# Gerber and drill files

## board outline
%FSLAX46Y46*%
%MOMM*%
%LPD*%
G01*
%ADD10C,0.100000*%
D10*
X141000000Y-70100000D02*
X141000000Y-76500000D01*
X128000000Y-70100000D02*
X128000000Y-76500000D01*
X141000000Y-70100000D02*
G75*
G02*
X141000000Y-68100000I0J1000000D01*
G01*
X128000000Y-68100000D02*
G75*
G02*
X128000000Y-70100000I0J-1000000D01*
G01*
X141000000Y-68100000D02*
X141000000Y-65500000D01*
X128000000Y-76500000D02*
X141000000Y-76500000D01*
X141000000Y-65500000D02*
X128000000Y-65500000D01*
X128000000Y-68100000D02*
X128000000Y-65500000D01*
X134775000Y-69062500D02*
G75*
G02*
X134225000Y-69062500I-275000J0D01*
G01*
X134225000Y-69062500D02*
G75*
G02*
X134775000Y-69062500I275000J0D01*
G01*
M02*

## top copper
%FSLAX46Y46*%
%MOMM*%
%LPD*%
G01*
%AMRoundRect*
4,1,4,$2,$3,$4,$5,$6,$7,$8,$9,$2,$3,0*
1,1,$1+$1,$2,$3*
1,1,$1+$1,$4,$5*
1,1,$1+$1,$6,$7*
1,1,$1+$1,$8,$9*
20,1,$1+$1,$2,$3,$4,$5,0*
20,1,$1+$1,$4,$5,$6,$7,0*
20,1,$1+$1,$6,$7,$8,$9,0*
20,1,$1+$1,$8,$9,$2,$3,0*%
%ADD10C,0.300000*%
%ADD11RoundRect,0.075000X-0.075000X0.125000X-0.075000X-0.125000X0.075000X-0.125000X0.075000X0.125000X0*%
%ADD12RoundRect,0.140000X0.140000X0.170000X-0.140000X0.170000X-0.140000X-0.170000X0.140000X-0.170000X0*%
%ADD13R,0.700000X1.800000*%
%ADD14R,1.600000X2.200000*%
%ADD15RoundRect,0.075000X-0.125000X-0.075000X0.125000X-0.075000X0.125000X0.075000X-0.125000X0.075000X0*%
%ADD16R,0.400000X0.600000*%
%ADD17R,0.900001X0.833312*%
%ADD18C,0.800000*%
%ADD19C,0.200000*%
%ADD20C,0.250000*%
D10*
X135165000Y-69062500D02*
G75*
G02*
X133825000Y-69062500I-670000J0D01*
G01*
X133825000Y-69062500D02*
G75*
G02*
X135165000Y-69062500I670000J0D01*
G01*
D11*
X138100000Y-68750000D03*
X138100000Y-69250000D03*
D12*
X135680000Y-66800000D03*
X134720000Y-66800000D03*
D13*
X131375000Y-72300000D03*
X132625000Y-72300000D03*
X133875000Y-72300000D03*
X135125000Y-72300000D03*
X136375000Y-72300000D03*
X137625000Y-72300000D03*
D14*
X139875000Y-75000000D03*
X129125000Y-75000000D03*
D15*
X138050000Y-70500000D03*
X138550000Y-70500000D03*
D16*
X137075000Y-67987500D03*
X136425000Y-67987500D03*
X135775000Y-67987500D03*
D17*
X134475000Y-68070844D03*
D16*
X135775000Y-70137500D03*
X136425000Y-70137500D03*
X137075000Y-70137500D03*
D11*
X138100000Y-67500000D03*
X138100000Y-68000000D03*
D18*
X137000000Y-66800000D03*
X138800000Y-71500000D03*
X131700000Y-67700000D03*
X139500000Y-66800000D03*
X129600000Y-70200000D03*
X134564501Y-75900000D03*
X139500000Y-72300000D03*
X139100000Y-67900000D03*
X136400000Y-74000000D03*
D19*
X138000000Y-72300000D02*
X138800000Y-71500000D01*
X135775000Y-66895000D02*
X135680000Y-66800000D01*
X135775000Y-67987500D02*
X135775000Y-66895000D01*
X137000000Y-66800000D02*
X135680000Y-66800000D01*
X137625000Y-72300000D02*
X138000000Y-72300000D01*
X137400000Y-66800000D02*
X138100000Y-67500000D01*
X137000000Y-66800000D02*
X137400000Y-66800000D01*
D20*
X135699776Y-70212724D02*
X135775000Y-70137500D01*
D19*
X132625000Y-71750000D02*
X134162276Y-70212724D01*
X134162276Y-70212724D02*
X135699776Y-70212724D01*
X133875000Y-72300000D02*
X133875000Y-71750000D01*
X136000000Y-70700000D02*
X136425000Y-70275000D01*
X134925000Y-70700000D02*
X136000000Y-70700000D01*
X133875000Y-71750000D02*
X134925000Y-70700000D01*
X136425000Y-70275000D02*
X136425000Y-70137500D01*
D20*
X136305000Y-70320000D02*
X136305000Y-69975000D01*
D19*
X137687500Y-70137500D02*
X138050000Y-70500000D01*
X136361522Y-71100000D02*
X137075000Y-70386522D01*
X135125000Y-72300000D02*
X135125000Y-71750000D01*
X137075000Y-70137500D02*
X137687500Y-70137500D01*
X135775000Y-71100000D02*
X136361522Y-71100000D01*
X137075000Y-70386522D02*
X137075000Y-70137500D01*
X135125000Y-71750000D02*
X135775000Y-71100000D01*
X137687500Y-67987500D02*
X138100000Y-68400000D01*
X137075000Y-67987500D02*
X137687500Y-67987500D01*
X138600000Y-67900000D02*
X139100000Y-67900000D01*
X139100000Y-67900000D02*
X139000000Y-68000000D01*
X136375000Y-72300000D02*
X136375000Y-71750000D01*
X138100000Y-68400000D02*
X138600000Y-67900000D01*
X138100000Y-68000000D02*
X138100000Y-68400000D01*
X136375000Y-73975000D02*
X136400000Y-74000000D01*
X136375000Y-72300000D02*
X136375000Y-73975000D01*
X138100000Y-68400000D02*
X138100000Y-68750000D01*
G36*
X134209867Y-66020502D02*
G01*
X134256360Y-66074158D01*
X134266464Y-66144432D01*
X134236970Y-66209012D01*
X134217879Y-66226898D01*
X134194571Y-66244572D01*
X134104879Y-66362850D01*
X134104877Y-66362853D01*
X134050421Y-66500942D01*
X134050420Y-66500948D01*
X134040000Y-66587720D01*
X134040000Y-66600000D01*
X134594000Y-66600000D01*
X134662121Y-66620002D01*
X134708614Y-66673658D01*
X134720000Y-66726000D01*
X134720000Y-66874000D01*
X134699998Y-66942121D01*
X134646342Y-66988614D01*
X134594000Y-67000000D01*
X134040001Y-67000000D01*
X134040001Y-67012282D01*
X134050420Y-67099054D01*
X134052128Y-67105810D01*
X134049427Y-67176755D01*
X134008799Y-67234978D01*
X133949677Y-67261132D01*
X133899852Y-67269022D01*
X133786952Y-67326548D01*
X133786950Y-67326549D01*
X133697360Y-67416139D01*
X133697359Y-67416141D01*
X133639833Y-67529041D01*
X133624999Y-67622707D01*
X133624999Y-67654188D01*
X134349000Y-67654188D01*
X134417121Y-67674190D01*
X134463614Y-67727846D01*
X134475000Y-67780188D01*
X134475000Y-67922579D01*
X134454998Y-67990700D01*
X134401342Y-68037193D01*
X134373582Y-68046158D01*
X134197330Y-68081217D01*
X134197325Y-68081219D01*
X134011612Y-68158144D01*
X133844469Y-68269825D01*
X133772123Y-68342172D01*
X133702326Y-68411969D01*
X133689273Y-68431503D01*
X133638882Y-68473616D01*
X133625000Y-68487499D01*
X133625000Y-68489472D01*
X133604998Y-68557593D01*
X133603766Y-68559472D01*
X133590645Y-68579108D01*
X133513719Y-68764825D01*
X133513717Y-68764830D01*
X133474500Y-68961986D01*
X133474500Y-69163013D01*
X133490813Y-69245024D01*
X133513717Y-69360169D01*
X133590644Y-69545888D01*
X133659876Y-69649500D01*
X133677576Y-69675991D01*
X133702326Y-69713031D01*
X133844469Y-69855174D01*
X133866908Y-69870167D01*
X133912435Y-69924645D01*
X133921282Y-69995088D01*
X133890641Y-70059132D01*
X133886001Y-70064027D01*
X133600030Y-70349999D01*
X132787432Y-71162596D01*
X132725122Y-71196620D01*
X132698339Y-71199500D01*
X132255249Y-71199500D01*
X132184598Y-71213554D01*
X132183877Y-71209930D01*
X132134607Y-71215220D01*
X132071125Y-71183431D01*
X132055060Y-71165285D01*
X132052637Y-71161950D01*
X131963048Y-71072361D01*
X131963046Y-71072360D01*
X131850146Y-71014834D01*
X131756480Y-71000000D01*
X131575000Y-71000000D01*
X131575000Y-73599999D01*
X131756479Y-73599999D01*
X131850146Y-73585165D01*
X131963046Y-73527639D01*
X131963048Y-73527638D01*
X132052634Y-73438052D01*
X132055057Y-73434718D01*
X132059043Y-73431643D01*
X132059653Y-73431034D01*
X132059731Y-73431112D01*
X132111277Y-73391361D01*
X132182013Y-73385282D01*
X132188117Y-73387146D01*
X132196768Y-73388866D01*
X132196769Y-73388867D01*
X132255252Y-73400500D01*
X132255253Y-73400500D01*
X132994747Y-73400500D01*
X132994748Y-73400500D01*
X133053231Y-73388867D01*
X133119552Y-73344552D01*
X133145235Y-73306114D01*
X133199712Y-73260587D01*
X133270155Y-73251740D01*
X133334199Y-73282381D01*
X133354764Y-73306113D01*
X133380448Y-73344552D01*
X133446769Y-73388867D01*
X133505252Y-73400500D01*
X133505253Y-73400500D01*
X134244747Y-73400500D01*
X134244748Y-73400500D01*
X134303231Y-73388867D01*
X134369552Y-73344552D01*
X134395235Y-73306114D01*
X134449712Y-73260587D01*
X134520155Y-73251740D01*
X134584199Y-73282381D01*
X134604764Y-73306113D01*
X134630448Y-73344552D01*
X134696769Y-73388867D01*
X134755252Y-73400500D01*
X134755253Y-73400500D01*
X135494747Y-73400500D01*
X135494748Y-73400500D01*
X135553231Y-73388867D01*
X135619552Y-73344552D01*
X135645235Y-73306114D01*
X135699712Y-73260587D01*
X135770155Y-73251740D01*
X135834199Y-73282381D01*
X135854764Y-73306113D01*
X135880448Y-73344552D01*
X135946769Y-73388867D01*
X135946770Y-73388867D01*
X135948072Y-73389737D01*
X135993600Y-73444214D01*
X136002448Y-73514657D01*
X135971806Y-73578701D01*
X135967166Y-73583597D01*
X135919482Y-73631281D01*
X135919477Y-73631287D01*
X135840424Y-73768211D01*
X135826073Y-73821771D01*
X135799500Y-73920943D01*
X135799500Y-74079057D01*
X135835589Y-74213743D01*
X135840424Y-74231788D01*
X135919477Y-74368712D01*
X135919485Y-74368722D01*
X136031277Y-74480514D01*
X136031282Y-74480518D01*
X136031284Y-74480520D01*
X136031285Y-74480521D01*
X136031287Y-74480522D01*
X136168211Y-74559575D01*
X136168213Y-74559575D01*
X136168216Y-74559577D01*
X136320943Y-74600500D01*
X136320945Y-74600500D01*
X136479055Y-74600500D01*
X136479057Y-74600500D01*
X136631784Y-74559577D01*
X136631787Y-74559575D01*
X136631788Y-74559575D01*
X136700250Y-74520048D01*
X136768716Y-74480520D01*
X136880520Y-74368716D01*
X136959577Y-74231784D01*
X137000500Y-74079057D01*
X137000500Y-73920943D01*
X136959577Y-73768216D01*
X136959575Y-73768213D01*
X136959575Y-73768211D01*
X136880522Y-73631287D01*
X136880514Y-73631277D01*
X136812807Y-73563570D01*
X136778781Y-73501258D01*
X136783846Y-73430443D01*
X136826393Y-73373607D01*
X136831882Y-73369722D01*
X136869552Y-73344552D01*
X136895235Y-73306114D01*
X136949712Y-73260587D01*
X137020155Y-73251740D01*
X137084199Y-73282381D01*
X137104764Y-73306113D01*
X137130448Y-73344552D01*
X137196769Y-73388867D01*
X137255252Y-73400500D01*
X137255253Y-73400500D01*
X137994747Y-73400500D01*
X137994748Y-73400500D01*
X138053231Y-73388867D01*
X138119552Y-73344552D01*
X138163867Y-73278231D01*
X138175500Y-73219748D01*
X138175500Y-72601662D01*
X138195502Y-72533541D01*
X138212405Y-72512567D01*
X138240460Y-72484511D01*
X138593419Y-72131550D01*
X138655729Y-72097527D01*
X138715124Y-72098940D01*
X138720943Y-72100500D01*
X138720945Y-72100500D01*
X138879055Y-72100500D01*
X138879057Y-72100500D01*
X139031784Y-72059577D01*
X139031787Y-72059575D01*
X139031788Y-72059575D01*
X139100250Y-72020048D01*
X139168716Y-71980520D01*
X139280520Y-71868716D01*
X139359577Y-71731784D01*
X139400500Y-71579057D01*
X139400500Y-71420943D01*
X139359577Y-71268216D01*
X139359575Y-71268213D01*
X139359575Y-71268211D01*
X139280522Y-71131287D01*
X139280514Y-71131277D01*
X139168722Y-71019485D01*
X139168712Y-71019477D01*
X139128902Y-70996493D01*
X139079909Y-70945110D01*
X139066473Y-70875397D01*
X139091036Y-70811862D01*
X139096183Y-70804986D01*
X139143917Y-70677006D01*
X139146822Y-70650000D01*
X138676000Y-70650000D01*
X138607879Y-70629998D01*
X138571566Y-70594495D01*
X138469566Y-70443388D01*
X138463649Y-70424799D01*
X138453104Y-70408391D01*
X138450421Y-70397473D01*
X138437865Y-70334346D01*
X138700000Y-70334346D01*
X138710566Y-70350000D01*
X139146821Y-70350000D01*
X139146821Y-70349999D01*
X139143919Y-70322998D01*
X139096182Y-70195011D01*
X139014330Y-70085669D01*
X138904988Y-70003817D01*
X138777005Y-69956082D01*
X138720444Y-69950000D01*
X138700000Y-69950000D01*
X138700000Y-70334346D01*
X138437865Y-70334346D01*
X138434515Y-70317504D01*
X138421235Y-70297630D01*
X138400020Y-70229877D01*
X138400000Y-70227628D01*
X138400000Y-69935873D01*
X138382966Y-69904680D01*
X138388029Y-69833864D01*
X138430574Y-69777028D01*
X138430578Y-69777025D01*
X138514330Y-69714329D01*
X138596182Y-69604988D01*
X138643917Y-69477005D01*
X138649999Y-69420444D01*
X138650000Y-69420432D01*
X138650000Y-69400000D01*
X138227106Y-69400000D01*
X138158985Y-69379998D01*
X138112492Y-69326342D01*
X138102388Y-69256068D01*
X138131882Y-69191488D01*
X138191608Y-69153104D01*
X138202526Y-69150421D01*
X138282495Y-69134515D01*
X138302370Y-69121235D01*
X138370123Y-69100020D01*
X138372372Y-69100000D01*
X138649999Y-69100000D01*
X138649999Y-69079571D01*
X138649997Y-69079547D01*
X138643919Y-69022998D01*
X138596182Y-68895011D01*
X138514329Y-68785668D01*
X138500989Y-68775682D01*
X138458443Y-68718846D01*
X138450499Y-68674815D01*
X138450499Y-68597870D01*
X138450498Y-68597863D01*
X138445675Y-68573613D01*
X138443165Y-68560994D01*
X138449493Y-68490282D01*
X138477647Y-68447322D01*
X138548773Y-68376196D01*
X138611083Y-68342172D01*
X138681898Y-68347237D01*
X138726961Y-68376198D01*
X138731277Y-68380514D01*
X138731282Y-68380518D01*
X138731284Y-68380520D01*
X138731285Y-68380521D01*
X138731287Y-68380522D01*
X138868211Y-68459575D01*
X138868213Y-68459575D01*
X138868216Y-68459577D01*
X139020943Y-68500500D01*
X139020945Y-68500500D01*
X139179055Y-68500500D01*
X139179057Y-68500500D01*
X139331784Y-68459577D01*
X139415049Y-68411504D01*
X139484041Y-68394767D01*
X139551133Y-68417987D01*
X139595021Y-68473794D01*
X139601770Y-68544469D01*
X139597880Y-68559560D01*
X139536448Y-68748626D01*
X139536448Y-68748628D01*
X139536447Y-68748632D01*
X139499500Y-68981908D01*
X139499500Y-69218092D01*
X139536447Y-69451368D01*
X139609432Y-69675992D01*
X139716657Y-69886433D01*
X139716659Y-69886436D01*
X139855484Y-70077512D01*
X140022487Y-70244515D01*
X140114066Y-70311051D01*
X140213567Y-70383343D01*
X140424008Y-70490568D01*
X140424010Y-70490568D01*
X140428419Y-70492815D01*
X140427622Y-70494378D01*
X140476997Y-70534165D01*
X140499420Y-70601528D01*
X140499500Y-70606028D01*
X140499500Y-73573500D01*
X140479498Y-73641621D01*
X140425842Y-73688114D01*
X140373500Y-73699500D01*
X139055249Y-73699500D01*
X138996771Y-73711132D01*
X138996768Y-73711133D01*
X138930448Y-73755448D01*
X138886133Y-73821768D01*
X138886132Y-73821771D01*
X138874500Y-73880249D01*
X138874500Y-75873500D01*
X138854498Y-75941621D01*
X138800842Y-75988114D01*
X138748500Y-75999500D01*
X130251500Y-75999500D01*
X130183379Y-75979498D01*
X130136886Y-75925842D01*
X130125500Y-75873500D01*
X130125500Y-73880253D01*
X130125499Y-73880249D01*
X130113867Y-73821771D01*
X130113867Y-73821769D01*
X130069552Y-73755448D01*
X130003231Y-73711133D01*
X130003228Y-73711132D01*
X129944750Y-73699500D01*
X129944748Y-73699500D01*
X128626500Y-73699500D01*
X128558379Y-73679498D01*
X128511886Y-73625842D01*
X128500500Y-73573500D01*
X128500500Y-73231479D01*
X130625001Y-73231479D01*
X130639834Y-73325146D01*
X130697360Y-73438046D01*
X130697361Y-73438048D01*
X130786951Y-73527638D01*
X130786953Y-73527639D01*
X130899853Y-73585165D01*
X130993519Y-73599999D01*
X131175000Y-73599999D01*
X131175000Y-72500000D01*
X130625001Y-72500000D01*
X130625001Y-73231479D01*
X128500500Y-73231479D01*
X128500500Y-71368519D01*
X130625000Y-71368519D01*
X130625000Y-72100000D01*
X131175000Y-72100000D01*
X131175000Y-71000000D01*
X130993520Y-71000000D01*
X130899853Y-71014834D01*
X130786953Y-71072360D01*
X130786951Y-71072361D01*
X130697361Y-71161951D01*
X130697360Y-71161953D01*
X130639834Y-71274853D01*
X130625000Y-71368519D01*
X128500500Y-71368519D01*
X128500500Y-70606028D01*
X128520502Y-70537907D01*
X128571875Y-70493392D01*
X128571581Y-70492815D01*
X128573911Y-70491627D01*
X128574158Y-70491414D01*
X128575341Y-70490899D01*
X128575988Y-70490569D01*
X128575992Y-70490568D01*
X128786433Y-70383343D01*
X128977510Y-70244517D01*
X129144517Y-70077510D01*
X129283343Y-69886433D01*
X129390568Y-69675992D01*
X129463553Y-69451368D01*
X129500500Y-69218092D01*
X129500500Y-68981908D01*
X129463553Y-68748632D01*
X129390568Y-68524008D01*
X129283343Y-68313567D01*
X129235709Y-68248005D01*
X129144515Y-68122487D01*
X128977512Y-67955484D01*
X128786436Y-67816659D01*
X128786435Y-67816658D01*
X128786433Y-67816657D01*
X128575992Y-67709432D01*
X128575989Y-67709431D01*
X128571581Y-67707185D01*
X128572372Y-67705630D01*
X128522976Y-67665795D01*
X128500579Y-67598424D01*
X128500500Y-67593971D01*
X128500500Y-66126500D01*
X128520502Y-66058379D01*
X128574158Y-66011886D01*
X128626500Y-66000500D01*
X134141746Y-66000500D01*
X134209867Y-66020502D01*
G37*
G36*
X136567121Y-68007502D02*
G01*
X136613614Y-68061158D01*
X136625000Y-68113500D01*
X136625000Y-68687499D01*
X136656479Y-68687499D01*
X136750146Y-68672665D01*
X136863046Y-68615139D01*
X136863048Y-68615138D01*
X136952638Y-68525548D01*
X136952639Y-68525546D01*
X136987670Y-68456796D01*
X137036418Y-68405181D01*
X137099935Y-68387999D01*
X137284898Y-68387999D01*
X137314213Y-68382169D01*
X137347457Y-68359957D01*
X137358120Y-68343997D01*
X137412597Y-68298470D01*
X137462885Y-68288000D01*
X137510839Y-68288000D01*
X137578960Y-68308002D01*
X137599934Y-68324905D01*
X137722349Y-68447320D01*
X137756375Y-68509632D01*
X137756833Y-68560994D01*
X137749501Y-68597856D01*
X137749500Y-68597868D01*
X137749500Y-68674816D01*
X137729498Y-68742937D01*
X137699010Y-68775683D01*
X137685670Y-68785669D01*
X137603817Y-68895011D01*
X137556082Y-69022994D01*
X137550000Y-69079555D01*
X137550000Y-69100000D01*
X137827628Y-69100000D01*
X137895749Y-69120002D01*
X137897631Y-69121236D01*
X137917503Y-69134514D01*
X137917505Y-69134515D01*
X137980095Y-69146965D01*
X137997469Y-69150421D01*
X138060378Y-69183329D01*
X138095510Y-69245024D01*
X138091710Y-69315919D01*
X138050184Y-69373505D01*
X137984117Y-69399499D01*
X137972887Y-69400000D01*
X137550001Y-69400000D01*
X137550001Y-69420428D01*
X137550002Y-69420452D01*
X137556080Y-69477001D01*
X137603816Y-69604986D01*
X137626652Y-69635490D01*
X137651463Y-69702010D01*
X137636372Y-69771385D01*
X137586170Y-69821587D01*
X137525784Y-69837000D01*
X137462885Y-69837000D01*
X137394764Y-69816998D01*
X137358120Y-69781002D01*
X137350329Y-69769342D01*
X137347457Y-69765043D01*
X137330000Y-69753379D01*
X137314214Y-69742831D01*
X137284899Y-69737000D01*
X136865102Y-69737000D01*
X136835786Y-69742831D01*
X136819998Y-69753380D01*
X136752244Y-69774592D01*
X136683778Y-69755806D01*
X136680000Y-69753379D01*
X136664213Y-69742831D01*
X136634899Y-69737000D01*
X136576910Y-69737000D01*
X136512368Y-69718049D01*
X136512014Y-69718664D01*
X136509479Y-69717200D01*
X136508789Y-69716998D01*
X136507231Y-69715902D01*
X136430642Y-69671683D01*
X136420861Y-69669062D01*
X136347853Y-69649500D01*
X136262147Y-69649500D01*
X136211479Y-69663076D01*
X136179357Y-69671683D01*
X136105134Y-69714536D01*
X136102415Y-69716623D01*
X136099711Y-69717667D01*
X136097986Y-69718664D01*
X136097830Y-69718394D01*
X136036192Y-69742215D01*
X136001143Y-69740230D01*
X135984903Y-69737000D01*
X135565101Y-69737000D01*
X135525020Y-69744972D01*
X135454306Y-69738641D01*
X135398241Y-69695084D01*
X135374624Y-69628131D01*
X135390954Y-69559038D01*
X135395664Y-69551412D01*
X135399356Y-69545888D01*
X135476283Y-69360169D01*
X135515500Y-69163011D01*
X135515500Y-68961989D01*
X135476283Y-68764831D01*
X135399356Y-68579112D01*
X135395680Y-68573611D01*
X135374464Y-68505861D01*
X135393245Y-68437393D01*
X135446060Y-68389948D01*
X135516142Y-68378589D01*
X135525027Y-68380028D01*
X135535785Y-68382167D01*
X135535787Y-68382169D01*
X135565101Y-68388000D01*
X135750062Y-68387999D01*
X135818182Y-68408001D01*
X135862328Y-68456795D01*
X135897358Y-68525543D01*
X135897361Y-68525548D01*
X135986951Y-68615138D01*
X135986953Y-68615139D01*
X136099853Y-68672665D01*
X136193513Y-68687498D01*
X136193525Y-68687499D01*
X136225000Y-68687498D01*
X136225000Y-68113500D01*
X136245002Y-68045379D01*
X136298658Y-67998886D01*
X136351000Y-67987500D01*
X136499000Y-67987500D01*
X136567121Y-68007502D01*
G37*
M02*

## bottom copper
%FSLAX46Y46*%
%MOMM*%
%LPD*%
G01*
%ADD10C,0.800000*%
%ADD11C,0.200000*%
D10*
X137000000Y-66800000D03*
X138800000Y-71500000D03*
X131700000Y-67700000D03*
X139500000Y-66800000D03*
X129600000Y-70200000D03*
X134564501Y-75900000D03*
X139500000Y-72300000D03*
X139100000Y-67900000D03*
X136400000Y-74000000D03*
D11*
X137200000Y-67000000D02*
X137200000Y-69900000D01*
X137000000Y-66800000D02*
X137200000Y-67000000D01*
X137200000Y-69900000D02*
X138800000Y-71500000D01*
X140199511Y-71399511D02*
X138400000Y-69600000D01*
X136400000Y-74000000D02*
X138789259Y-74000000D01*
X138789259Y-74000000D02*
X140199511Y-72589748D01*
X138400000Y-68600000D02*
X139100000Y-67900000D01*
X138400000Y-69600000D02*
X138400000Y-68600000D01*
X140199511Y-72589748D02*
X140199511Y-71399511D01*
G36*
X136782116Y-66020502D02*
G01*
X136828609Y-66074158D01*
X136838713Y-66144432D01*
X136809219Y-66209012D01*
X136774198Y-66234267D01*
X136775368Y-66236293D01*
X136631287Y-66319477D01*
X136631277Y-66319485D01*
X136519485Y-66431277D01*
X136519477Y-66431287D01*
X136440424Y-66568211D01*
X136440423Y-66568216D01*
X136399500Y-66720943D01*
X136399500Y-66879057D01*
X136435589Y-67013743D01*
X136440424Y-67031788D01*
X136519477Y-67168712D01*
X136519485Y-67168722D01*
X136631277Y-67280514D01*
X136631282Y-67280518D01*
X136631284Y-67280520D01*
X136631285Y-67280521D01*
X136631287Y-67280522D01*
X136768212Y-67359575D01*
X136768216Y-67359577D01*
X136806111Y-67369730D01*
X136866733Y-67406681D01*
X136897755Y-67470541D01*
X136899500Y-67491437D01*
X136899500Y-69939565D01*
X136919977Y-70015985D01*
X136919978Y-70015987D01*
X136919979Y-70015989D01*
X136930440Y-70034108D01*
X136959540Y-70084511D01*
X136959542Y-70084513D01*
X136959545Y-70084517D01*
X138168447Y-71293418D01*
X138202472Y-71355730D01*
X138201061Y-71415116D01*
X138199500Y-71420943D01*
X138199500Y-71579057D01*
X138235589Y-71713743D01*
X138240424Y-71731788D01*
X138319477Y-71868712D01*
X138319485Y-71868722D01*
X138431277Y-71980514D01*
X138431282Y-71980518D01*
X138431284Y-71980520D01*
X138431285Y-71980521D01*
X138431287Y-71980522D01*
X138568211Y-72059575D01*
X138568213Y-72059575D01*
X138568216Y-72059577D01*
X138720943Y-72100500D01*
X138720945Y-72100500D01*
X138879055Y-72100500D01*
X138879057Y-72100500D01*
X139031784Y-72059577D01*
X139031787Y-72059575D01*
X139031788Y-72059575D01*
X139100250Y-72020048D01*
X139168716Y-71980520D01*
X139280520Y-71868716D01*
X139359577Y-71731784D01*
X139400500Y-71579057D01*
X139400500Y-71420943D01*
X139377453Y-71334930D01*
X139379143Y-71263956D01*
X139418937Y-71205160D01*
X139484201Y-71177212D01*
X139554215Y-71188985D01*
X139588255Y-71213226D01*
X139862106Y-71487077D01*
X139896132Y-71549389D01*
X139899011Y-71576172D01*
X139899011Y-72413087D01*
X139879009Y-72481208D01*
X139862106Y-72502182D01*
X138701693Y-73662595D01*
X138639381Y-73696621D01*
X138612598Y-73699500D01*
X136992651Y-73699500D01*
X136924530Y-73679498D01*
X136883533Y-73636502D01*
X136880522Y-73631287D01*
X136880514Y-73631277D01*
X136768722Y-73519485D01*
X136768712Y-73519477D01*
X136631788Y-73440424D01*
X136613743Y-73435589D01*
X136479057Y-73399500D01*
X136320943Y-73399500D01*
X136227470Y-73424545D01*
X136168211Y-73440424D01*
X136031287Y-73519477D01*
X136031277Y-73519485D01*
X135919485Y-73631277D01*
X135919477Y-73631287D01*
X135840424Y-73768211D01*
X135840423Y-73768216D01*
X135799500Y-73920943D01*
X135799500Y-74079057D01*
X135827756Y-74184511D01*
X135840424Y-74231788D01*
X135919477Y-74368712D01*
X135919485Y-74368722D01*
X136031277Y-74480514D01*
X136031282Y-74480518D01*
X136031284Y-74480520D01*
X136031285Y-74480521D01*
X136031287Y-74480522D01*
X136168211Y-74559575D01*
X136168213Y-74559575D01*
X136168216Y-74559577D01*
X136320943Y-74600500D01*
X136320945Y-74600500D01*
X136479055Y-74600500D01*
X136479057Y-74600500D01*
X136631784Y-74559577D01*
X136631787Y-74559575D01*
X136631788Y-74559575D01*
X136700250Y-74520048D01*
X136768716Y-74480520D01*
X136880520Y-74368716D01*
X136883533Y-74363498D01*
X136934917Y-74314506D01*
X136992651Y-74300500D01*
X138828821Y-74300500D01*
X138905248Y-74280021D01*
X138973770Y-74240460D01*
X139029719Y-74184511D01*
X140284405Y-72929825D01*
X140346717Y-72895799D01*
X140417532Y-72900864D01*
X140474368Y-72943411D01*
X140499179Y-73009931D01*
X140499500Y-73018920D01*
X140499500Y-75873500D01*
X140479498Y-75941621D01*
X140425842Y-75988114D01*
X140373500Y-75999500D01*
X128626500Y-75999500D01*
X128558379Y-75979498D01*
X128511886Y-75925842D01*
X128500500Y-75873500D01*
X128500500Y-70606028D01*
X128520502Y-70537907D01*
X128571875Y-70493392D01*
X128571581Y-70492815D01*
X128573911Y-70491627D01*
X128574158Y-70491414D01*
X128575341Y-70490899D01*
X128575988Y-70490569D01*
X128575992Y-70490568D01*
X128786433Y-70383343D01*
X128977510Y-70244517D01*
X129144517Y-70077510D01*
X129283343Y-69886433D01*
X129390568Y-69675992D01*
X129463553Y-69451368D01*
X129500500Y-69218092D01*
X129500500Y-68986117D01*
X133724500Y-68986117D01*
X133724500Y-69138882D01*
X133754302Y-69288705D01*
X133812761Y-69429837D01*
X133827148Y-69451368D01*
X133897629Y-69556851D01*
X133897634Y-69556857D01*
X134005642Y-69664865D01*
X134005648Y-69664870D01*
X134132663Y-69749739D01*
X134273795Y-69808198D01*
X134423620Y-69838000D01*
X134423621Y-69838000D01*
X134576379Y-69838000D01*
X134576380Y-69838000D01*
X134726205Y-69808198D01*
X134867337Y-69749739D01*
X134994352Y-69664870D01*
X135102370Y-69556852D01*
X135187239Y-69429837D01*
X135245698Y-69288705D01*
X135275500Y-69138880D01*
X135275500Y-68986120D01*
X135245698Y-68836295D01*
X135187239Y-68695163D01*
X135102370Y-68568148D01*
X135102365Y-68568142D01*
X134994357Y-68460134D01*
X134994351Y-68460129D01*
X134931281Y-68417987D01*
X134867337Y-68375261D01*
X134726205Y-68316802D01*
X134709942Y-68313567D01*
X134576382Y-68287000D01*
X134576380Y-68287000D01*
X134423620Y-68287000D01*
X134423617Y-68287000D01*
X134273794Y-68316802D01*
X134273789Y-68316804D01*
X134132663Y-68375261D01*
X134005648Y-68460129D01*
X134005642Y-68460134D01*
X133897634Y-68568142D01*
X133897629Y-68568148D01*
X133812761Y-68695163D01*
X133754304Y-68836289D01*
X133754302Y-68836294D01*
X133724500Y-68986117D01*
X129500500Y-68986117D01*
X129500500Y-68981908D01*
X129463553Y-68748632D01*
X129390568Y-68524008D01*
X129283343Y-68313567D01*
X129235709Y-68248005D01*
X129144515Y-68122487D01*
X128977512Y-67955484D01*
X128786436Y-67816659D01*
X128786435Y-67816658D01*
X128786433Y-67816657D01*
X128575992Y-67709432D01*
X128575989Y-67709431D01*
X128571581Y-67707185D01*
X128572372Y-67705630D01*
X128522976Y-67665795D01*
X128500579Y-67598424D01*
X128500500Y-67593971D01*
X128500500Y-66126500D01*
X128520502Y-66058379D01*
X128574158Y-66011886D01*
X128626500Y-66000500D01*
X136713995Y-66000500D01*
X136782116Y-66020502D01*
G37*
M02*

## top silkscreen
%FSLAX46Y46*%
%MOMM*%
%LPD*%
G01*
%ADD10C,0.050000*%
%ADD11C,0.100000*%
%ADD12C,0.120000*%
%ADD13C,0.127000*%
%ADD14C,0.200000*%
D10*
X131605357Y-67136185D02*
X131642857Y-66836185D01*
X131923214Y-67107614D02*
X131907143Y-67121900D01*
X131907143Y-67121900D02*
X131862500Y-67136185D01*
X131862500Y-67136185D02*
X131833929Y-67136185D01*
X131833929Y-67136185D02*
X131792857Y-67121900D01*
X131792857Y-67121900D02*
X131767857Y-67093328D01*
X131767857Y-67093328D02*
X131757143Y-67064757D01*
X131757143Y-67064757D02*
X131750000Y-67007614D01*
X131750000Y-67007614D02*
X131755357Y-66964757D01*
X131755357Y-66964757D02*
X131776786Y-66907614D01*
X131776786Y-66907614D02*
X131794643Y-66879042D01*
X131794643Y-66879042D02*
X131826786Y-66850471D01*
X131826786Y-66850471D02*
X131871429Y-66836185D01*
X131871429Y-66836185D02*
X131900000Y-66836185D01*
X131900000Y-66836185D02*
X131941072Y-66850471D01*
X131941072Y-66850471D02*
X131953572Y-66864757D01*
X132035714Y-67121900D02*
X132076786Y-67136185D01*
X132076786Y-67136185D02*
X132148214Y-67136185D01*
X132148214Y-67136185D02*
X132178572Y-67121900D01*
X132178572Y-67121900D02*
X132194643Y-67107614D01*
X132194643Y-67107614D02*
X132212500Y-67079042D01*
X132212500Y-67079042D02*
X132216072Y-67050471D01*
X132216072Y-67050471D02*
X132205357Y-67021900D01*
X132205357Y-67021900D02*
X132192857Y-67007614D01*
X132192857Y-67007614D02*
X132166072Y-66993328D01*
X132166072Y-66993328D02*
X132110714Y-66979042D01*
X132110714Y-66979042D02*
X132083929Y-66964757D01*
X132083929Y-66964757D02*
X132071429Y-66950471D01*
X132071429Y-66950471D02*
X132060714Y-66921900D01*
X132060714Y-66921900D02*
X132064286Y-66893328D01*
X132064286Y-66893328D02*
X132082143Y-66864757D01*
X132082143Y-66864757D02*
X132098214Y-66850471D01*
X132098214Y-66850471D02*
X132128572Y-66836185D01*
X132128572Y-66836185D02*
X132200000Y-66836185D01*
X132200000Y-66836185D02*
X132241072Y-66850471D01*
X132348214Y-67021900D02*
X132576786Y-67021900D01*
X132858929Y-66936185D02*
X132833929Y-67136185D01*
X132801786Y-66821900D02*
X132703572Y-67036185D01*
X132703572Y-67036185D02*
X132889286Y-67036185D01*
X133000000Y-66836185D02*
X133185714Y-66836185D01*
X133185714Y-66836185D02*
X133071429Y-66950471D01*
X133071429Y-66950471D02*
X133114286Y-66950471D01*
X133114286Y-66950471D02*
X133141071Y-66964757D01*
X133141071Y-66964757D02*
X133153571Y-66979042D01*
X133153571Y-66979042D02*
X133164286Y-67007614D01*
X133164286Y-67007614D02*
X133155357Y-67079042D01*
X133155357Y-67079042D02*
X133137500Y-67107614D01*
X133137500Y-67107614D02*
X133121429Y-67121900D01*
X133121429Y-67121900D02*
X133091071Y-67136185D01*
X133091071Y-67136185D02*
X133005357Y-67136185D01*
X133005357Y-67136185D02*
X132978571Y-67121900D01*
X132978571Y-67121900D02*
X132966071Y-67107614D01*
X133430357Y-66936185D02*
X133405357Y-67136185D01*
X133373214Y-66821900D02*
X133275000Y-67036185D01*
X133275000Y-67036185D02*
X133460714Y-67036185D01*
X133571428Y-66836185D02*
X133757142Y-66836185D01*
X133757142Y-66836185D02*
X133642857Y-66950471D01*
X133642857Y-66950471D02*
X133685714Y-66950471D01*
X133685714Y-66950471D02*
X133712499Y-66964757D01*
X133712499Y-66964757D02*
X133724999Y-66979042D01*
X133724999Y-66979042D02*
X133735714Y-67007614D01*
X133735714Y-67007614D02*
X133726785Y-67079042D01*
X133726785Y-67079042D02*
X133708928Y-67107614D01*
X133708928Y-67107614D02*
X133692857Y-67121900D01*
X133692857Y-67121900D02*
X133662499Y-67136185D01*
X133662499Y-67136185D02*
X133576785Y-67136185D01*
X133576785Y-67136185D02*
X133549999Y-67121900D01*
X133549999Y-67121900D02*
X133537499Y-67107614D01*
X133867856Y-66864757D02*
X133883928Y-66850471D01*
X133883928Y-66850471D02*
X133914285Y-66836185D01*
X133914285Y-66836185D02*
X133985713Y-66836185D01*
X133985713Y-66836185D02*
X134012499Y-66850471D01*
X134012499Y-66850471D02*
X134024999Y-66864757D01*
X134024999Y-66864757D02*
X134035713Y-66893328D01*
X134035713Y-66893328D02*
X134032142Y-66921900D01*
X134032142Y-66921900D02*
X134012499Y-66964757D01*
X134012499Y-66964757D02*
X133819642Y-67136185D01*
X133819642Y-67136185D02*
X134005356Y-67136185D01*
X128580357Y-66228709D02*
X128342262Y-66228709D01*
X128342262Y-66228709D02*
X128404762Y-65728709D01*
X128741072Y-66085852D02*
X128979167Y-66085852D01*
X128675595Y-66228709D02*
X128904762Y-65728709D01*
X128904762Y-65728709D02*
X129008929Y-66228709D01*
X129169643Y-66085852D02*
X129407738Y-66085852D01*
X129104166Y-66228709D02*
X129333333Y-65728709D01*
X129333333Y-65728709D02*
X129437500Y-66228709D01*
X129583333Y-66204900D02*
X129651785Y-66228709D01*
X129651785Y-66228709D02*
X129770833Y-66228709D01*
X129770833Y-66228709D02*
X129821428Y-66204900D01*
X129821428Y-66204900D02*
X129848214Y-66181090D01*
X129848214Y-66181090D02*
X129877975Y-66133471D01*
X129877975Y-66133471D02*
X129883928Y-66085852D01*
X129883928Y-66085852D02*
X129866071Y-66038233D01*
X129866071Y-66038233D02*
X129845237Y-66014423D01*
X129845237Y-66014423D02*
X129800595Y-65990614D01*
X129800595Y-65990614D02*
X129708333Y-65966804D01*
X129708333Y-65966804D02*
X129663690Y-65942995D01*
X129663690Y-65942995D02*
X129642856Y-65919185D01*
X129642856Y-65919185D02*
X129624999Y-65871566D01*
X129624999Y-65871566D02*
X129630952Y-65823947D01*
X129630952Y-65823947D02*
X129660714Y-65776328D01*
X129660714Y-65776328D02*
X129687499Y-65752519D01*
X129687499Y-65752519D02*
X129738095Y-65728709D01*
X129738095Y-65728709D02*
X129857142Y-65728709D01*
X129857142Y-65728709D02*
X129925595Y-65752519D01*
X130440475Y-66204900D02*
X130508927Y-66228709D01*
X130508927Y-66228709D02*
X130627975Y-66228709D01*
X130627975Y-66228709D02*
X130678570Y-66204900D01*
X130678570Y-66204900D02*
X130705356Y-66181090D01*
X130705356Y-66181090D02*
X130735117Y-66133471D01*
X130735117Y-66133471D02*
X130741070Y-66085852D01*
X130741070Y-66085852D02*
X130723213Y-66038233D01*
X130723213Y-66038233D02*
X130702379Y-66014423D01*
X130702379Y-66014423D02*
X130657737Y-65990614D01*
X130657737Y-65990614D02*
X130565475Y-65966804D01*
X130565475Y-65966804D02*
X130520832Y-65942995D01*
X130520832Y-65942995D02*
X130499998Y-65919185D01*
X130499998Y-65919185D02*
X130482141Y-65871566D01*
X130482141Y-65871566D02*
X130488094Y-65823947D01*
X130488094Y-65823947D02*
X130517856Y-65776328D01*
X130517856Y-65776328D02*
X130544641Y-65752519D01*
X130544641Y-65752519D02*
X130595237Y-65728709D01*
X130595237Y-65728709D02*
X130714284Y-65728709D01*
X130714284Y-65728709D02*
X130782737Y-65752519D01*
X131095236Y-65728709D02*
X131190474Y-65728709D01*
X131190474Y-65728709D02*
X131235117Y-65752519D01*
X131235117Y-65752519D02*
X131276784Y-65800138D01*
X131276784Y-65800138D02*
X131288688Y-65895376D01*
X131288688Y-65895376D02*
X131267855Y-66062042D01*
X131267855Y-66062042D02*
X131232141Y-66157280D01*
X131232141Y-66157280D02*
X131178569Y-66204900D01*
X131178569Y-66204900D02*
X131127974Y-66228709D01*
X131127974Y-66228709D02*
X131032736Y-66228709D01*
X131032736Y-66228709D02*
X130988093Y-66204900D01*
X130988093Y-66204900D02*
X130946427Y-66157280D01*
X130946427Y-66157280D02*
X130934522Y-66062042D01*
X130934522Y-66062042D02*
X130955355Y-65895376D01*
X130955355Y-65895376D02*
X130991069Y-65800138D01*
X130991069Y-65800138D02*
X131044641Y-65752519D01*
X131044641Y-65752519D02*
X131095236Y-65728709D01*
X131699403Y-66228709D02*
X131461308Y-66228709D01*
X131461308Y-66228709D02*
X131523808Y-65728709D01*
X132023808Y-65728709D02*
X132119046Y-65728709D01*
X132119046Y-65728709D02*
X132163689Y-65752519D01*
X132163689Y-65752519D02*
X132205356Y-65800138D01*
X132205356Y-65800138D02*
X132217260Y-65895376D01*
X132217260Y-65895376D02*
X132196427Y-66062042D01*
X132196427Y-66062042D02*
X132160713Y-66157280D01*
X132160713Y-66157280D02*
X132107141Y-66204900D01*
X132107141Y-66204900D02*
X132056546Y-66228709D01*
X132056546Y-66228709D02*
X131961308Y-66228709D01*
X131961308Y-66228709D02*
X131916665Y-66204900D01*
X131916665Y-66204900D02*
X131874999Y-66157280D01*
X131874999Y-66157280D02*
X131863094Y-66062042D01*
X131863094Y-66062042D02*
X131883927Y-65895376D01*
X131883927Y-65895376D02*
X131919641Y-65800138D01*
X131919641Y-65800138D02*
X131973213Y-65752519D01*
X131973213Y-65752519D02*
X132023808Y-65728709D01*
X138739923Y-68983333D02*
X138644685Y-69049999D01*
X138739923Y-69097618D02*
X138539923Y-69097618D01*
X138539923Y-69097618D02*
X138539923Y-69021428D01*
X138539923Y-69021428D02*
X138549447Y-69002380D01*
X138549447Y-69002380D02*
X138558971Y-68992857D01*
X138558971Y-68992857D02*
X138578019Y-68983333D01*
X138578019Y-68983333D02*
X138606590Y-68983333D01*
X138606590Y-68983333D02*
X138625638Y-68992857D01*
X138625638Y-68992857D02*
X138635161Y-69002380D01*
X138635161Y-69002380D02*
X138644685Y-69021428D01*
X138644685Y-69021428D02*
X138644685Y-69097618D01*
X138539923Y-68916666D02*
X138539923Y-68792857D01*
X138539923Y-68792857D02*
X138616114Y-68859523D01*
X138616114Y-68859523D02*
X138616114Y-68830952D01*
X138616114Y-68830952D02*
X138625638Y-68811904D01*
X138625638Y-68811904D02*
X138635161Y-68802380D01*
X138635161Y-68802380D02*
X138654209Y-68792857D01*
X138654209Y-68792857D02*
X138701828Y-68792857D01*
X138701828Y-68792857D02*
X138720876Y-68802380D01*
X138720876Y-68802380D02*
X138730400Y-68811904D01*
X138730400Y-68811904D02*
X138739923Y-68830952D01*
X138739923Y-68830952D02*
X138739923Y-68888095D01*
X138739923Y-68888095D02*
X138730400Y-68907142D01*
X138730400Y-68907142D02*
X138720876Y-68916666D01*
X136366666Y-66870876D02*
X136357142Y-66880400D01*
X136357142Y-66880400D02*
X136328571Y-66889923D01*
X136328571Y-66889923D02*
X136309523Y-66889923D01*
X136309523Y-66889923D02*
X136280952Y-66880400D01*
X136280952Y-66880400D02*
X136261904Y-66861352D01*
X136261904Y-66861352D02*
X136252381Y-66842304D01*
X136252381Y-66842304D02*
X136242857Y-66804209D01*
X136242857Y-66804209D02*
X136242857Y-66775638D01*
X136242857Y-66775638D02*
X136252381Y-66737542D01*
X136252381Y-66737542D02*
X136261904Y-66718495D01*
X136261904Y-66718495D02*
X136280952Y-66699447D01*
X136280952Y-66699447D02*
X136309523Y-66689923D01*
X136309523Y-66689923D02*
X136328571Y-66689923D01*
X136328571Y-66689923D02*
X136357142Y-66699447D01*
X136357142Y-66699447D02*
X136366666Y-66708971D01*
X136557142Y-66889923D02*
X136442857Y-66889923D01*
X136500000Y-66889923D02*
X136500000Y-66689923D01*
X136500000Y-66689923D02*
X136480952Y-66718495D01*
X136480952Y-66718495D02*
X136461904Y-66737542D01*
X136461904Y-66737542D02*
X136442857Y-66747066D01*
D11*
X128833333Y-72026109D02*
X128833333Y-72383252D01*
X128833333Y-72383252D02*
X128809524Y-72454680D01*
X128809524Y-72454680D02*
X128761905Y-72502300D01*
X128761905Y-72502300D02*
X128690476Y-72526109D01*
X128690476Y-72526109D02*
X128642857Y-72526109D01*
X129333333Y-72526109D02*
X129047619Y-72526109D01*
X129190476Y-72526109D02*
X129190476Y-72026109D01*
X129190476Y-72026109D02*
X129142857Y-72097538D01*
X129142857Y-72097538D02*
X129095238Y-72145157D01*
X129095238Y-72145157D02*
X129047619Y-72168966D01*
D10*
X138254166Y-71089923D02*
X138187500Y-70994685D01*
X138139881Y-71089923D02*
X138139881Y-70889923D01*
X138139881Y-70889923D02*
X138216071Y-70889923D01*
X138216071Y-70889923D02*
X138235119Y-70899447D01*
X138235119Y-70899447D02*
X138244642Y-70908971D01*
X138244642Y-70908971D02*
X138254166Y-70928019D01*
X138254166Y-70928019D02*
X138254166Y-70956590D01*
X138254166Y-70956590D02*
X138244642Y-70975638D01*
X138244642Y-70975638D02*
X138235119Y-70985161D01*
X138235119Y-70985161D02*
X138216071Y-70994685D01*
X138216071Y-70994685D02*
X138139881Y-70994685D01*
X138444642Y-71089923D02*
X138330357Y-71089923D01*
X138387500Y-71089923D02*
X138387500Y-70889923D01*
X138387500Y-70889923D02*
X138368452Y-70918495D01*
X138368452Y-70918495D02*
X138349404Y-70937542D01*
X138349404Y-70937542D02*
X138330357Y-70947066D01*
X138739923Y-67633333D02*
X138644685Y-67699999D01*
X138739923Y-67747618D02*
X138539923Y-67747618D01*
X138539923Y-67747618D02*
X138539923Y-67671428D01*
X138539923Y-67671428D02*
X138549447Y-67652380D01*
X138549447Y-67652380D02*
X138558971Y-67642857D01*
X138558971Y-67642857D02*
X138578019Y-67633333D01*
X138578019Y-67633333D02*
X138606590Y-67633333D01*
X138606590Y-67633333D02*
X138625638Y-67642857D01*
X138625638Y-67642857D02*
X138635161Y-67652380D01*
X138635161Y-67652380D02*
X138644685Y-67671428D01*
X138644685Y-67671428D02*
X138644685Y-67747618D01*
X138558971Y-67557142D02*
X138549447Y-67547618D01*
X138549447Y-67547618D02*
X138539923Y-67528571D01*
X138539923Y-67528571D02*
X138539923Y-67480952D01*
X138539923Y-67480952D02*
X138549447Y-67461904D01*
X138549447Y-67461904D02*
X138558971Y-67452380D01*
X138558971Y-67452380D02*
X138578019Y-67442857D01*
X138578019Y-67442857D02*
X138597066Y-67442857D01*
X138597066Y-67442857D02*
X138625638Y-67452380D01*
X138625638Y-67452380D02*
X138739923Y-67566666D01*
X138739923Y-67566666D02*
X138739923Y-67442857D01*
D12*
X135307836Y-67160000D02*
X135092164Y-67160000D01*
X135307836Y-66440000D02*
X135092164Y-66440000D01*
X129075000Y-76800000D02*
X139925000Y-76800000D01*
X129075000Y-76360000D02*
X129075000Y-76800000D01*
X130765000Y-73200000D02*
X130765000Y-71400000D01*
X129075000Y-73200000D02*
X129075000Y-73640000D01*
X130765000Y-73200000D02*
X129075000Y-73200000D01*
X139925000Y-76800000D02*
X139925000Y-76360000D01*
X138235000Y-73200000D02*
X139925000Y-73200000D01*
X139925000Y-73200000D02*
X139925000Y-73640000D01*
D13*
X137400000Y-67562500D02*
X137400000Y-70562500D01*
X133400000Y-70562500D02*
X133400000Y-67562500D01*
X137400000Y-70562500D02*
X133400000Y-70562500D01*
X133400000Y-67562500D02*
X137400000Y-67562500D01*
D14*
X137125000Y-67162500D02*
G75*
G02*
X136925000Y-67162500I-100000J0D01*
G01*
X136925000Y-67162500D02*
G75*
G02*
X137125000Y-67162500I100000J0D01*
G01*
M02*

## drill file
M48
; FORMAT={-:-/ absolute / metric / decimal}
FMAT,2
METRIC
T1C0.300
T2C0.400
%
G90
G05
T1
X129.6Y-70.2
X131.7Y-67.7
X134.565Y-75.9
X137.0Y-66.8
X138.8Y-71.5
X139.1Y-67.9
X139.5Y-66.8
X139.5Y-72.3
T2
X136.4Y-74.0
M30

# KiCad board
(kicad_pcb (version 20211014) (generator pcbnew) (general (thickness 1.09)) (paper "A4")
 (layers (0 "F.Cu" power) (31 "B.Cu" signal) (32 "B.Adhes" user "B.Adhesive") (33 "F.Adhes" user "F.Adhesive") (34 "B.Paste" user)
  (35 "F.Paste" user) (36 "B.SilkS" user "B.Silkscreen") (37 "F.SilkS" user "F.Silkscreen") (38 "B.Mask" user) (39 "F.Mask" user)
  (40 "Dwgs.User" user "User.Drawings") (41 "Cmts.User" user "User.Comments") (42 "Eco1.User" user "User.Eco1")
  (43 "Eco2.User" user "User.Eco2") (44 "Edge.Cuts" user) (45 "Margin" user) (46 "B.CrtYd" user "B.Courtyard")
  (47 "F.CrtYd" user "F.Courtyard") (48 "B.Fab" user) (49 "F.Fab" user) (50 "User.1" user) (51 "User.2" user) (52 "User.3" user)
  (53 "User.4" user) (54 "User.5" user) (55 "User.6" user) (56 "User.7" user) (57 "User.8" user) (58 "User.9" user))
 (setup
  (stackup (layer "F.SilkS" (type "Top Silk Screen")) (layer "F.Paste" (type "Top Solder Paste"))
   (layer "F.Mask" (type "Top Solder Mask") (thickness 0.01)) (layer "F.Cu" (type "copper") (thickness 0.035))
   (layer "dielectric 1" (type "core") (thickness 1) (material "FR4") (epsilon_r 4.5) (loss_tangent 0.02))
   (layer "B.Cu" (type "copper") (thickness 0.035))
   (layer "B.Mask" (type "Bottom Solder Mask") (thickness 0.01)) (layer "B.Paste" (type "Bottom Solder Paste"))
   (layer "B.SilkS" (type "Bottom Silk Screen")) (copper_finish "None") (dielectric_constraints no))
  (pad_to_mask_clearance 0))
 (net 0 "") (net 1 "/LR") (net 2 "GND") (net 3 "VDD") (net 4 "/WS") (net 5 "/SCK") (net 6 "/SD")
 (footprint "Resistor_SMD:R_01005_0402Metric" (layer "F.Cu") (at 138.1 69 -90)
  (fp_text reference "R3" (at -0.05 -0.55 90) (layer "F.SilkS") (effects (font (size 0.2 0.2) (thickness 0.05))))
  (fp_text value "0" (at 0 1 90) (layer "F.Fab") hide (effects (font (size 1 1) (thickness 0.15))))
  (pad "" smd roundrect (at -0.275 0 270) (size 0.27 0.27) (layers "F.Paste") (roundrect_rratio 0.25))
  (pad "" smd roundrect (at 0.275 0 270) (size 0.27 0.27) (layers "F.Paste") (roundrect_rratio 0.25))
  (pad "1" smd roundrect (at -0.25 0 270) (size 0.4 0.3) (layers "F.Cu" "F.Mask") (roundrect_rratio 0.25) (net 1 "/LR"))
  (pad "2" smd roundrect (at 0.25 0 270) (size 0.4 0.3) (layers "F.Cu" "F.Mask") (roundrect_rratio 0.25) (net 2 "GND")))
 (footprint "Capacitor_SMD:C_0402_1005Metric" (layer "F.Cu") (at 135.2 66.8 180)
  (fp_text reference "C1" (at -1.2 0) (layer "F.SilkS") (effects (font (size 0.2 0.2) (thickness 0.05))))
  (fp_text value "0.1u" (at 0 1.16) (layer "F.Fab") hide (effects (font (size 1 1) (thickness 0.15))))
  (fp_line (start -0.107836 -0.36) (end 0.107836 -0.36) (layer "F.SilkS") (width 0.12))
  (fp_line (start -0.107836 0.36) (end 0.107836 0.36) (layer "F.SilkS") (width 0.12))
  (pad "1" smd roundrect (at -0.48 0 180) (size 0.56 0.62) (layers "F.Cu" "F.Paste" "F.Mask") (roundrect_rratio 0.25) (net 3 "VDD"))
  (pad "2" smd roundrect (at 0.48 0 180) (size 0.56 0.62) (layers "F.Cu" "F.Paste" "F.Mask") (roundrect_rratio 0.25) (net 2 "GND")))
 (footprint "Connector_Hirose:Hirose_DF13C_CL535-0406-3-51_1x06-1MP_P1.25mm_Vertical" (layer "F.Cu") (at 134.5 73.75)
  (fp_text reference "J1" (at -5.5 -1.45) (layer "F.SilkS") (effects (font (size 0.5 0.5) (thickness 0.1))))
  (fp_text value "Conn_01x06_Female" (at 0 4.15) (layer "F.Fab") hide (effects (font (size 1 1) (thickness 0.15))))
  (fp_line (start -5.425 3.05) (end 5.425 3.05) (layer "F.SilkS") (width 0.12))
  (fp_line (start -5.425 2.61) (end -5.425 3.05) (layer "F.SilkS") (width 0.12))
  (fp_line (start -3.735 -0.55) (end -3.735 -2.35) (layer "F.SilkS") (width 0.12))
  (fp_line (start -5.425 -0.55) (end -5.425 -0.11) (layer "F.SilkS") (width 0.12))
  (fp_line (start -3.735 -0.55) (end -5.425 -0.55) (layer "F.SilkS") (width 0.12))
  (fp_line (start 5.425 3.05) (end 5.425 2.61) (layer "F.SilkS") (width 0.12))
  (fp_line (start 3.735 -0.55) (end 5.425 -0.55) (layer "F.SilkS") (width 0.12))
  (fp_line (start 5.425 -0.55) (end 5.425 -0.11) (layer "F.SilkS") (width 0.12))
  (pad "1" smd rect locked (at -3.125 -1.45) (size 0.7 1.8) (layers "F.Cu" "F.Paste" "F.Mask") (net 2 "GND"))
  (pad "2" smd rect locked (at -1.875 -1.45) (size 0.7 1.8) (layers "F.Cu" "F.Paste" "F.Mask") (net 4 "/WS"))
  (pad "3" smd rect locked (at -0.625 -1.45) (size 0.7 1.8) (layers "F.Cu" "F.Paste" "F.Mask") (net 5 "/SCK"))
  (pad "4" smd rect locked (at 0.625 -1.45) (size 0.7 1.8) (layers "F.Cu" "F.Paste" "F.Mask") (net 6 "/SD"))
  (pad "5" smd rect locked (at 1.875 -1.45) (size 0.7 1.8) (layers "F.Cu" "F.Paste" "F.Mask") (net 1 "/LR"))
  (pad "6" smd rect locked (at 3.125 -1.45) (size 0.7 1.8) (layers "F.Cu" "F.Paste" "F.Mask") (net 3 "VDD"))
  (pad "MP" smd rect locked (at 5.375 1.25) (size 1.6 2.2) (layers "F.Cu" "F.Paste" "F.Mask"))
  (pad "MP" smd rect locked (at -5.375 1.25) (size 1.6 2.2) (layers "F.Cu" "F.Paste" "F.Mask")))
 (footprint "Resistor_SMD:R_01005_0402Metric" (layer "F.Cu") (at 138.3 70.5)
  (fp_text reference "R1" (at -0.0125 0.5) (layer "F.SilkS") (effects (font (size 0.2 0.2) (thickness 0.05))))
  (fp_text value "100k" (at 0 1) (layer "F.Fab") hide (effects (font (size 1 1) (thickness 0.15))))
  (pad "" smd roundrect (at -0.275 0) (size 0.27 0.27) (layers "F.Paste") (roundrect_rratio 0.25))
  (pad "" smd roundrect (at 0.275 0) (size 0.27 0.27) (layers "F.Paste") (roundrect_rratio 0.25))
  (pad "1" smd roundrect (at -0.25 0) (size 0.4 0.3) (layers "F.Cu" "F.Mask") (roundrect_rratio 0.25) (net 6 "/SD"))
  (pad "2" smd roundrect (at 0.25 0) (size 0.4 0.3) (layers "F.Cu" "F.Mask") (roundrect_rratio 0.25) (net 2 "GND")))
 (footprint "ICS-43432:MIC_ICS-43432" (layer "F.Cu") (at 135.4 69.0625 -90) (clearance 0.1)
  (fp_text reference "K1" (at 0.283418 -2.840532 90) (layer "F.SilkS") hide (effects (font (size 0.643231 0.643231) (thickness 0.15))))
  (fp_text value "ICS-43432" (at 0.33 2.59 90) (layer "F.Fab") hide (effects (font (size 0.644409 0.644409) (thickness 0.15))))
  (fp_circle (center 0 0.905) (end 0.67 0.905) (layer "F.Cu") (width 0.3) (fill none))
  (fp_line (start -1.5 -2) (end 1.5 -2) (layer "F.SilkS") (width 0.127))
  (fp_line (start 1.5 2) (end -1.5 2) (layer "F.SilkS") (width 0.127))
  (fp_line (start 1.5 -2) (end 1.5 2) (layer "F.SilkS") (width 0.127))
  (fp_line (start -1.5 2) (end -1.5 -2) (layer "F.SilkS") (width 0.127))
  (fp_circle (center -1.9 -1.625) (end -1.8 -1.625) (layer "F.SilkS") (width 0.2) (fill none))
  (fp_circle (center 0 0.9) (end 0.275 0.9) (layer "Edge.Cuts") (width 0.1) (fill none))
  (pad "1" smd rect (at -1.075 -1.675 270) (size 0.6 0.4) (layers "F.Cu" "F.Mask") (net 1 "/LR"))
  (pad "2" smd rect (at -1.075 -1.025 270) (size 0.6 0.4) (layers "F.Cu" "F.Mask") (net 2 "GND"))
  (pad "3" smd rect (at -1.075 -0.375 270) (size 0.6 0.4) (layers "F.Cu" "F.Mask") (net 3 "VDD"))
  (pad "4" smd rect (at -0.991656 0.925 270) (size 0.833312 0.900001) (layers "F.Cu") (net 2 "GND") (thermal_width 1))
  (pad "5" smd rect (at 1.075 -0.375 270) (size 0.6 0.4) (layers "F.Cu" "F.Mask") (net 4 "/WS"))
  (pad "6" smd rect (at 1.075 -1.025 270) (size 0.6 0.4) (layers "F.Cu" "F.Mask") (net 5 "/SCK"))
  (pad "7" smd rect (at 1.075 -1.675 270) (size 0.6 0.4) (layers "F.Cu" "F.Mask") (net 6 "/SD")))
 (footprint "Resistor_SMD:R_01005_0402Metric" (layer "F.Cu") (at 138.1 67.75 -90)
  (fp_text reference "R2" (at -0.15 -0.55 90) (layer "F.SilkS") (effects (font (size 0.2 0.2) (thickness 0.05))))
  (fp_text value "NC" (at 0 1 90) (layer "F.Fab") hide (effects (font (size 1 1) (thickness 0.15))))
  (pad "" smd roundrect (at -0.275 0 270) (size 0.27 0.27) (layers "F.Paste") (roundrect_rratio 0.25))
  (pad "" smd roundrect (at 0.275 0 270) (size 0.27 0.27) (layers "F.Paste") (roundrect_rratio 0.25))
  (pad "1" smd roundrect (at -0.25 0 270) (size 0.4 0.3) (layers "F.Cu" "F.Mask") (roundrect_rratio 0.25) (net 3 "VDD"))
  (pad "2" smd roundrect (at 0.25 0 270) (size 0.4 0.3) (layers "F.Cu" "F.Mask") (roundrect_rratio 0.25) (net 1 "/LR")))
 (gr_line (start 141 70.1) (end 141 76.5) (layer "Edge.Cuts") (width 0.1))
 (gr_line (start 128 70.1) (end 128 76.5) (layer "Edge.Cuts") (width 0.1))
 (gr_arc (start 141 70.1) (mid 140 69.1) (end 141 68.1) (layer "Edge.Cuts") (width 0.1))
 (gr_arc (start 128 68.1) (mid 129 69.1) (end 128 70.1) (layer "Edge.Cuts") (width 0.1))
 (gr_line (start 141 68.1) (end 141 65.5) (layer "Edge.Cuts") (width 0.1))
 (gr_line (start 128 76.5) (end 141 76.5) (layer "Edge.Cuts") (width 0.1))
 (gr_line (start 141 65.5) (end 128 65.5) (layer "Edge.Cuts") (width 0.1))
 (gr_line (start 128 68.1) (end 128 65.5) (layer "Edge.Cuts") (width 0.1))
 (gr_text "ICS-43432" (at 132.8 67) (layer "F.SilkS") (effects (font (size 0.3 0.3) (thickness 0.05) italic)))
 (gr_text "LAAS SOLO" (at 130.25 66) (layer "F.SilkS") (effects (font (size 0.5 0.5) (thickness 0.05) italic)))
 (segment (start 138 72.3) (end 138.8 71.5) (width 0.2) (layer "F.Cu") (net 3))
 (segment (start 135.775 66.895) (end 135.68 66.8) (width 0.2) (layer "F.Cu") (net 3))
 (segment (start 135.775 67.9875) (end 135.775 66.895) (width 0.2) (layer "F.Cu") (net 3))
 (segment (start 137 66.8) (end 135.68 66.8) (width 0.2) (layer "F.Cu") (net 3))
 (segment (start 137.625 72.3) (end 138 72.3) (width 0.2) (layer "F.Cu") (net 3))
 (segment (start 137.4 66.8) (end 138.1 67.5) (width 0.2) (layer "F.Cu") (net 3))
 (segment (start 137 66.8) (end 137.4 66.8) (width 0.2) (layer "F.Cu") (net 3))
 (via (at 137 66.8) (size 0.8) (drill 0.3) (layers "F.Cu" "B.Cu") (free) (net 3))
 (via (at 138.8 71.5) (size 0.8) (drill 0.3) (layers "F.Cu" "B.Cu") (free) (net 3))
 (segment (start 137.2 67) (end 137.2 69.9) (width 0.2) (layer "B.Cu") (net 3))
 (segment (start 137 66.8) (end 137.2 67) (width 0.2) (layer "B.Cu") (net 3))
 (segment (start 137.2 69.9) (end 138.8 71.5) (width 0.2) (layer "B.Cu") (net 3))
 (via (at 131.7 67.7) (size 0.8) (drill 0.3) (layers "F.Cu" "B.Cu") (free) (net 2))
 (via (at 139.5 66.8) (size 0.8) (drill 0.3) (layers "F.Cu" "B.Cu") (free) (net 2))
 (via (at 129.6 70.2) (size 0.8) (drill 0.3) (layers "F.Cu" "B.Cu") (free) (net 2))
 (via (at 134.564501 75.9) (size 0.8) (drill 0.3) (layers "F.Cu" "B.Cu") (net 2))
 (via (at 139.5 72.3) (size 0.8) (drill 0.3) (layers "F.Cu" "B.Cu") (free) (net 2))
 (segment (start 135.699776 70.212724) (end 135.775 70.1375) (width 0.25) (layer "F.Cu") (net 4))
 (segment (start 132.625 71.75) (end 134.162276 70.212724) (width 0.2) (layer "F.Cu") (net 4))
 (segment (start 134.162276 70.212724) (end 135.699776 70.212724) (width 0.2) (layer "F.Cu") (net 4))
 (segment (start 133.875 72.3) (end 133.875 71.75) (width 0.2) (layer "F.Cu") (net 5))
 (segment (start 136 70.7) (end 136.425 70.275) (width 0.2) (layer "F.Cu") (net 5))
 (segment (start 134.925 70.7) (end 136 70.7) (width 0.2) (layer "F.Cu") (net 5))
 (segment (start 133.875 71.75) (end 134.925 70.7) (width 0.2) (layer "F.Cu") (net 5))
 (segment (start 136.425 70.275) (end 136.425 70.1375) (width 0.2) (layer "F.Cu") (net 5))
 (segment (start 136.305 70.32) (end 136.305 69.975) (width 0.25) (layer "F.Cu") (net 5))
 (segment (start 137.6875 70.1375) (end 138.05 70.5) (width 0.2) (layer "F.Cu") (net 6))
 (segment (start 136.361522 71.1) (end 137.075 70.386522) (width 0.2) (layer "F.Cu") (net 6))
 (segment (start 135.125 72.3) (end 135.125 71.75) (width 0.2) (layer "F.Cu") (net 6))
 (segment (start 137.075 70.1375) (end 137.6875 70.1375) (width 0.2) (layer "F.Cu") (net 6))
 (segment (start 135.775 71.1) (end 136.361522 71.1) (width 0.2) (layer "F.Cu") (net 6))
 (segment (start 137.075 70.386522) (end 137.075 70.1375) (width 0.2) (layer "F.Cu") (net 6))
 (segment (start 135.125 71.75) (end 135.775 71.1) (width 0.2) (layer "F.Cu") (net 6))
 (segment (start 137.6875 67.9875) (end 138.1 68.4) (width 0.2) (layer "F.Cu") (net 1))
 (segment (start 137.075 67.9875) (end 137.6875 67.9875) (width 0.2) (layer "F.Cu") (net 1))
 (segment (start 138.6 67.9) (end 139.1 67.9) (width 0.2) (layer "F.Cu") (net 1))
 (segment (start 139.1 67.9) (end 139 68) (width 0.2) (layer "F.Cu") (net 1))
 (segment (start 136.375 72.3) (end 136.375 71.75) (width 0.2) (layer "F.Cu") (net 1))
 (segment (start 138.1 68.4) (end 138.6 67.9) (width 0.2) (layer "F.Cu") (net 1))
 (segment (start 138.1 68) (end 138.1 68.4) (width 0.2) (layer "F.Cu") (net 1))
 (segment (start 136.375 73.975) (end 136.4 74) (width 0.2) (layer "F.Cu") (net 1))
 (segment (start 136.375 72.3) (end 136.375 73.975) (width 0.2) (layer "F.Cu") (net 1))
 (segment (start 138.1 68.4) (end 138.1 68.75) (width 0.2) (layer "F.Cu") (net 1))
 (via (at 139.1 67.9) (size 0.8) (drill 0.3) (layers "F.Cu" "B.Cu") (free) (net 1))
 (via (at 136.4 74) (size 0.8) (drill 0.4) (layers "F.Cu" "B.Cu") (free) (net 1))
 (segment (start 140.199511 71.399511) (end 138.4 69.6) (width 0.2) (layer "B.Cu") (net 1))
 (segment (start 136.4 74) (end 138.789259 74) (width 0.2) (layer "B.Cu") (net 1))
 (segment (start 138.789259 74) (end 140.199511 72.589748) (width 0.2) (layer "B.Cu") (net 1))
 (segment (start 138.4 68.6) (end 139.1 67.9) (width 0.2) (layer "B.Cu") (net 1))
 (segment (start 138.4 69.6) (end 138.4 68.6) (width 0.2) (layer "B.Cu") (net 1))
 (segment (start 140.199511 72.589748) (end 140.199511 71.399511) (width 0.2) (layer "B.Cu") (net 1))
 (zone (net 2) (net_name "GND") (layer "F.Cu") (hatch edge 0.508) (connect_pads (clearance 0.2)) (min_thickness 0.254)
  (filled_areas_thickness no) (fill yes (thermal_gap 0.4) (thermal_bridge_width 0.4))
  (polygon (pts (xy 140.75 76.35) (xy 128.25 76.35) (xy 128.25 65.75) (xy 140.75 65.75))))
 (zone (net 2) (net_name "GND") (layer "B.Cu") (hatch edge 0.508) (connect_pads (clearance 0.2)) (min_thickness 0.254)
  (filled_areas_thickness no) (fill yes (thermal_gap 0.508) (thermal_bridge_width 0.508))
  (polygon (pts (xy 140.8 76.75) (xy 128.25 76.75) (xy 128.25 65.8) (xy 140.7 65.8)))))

